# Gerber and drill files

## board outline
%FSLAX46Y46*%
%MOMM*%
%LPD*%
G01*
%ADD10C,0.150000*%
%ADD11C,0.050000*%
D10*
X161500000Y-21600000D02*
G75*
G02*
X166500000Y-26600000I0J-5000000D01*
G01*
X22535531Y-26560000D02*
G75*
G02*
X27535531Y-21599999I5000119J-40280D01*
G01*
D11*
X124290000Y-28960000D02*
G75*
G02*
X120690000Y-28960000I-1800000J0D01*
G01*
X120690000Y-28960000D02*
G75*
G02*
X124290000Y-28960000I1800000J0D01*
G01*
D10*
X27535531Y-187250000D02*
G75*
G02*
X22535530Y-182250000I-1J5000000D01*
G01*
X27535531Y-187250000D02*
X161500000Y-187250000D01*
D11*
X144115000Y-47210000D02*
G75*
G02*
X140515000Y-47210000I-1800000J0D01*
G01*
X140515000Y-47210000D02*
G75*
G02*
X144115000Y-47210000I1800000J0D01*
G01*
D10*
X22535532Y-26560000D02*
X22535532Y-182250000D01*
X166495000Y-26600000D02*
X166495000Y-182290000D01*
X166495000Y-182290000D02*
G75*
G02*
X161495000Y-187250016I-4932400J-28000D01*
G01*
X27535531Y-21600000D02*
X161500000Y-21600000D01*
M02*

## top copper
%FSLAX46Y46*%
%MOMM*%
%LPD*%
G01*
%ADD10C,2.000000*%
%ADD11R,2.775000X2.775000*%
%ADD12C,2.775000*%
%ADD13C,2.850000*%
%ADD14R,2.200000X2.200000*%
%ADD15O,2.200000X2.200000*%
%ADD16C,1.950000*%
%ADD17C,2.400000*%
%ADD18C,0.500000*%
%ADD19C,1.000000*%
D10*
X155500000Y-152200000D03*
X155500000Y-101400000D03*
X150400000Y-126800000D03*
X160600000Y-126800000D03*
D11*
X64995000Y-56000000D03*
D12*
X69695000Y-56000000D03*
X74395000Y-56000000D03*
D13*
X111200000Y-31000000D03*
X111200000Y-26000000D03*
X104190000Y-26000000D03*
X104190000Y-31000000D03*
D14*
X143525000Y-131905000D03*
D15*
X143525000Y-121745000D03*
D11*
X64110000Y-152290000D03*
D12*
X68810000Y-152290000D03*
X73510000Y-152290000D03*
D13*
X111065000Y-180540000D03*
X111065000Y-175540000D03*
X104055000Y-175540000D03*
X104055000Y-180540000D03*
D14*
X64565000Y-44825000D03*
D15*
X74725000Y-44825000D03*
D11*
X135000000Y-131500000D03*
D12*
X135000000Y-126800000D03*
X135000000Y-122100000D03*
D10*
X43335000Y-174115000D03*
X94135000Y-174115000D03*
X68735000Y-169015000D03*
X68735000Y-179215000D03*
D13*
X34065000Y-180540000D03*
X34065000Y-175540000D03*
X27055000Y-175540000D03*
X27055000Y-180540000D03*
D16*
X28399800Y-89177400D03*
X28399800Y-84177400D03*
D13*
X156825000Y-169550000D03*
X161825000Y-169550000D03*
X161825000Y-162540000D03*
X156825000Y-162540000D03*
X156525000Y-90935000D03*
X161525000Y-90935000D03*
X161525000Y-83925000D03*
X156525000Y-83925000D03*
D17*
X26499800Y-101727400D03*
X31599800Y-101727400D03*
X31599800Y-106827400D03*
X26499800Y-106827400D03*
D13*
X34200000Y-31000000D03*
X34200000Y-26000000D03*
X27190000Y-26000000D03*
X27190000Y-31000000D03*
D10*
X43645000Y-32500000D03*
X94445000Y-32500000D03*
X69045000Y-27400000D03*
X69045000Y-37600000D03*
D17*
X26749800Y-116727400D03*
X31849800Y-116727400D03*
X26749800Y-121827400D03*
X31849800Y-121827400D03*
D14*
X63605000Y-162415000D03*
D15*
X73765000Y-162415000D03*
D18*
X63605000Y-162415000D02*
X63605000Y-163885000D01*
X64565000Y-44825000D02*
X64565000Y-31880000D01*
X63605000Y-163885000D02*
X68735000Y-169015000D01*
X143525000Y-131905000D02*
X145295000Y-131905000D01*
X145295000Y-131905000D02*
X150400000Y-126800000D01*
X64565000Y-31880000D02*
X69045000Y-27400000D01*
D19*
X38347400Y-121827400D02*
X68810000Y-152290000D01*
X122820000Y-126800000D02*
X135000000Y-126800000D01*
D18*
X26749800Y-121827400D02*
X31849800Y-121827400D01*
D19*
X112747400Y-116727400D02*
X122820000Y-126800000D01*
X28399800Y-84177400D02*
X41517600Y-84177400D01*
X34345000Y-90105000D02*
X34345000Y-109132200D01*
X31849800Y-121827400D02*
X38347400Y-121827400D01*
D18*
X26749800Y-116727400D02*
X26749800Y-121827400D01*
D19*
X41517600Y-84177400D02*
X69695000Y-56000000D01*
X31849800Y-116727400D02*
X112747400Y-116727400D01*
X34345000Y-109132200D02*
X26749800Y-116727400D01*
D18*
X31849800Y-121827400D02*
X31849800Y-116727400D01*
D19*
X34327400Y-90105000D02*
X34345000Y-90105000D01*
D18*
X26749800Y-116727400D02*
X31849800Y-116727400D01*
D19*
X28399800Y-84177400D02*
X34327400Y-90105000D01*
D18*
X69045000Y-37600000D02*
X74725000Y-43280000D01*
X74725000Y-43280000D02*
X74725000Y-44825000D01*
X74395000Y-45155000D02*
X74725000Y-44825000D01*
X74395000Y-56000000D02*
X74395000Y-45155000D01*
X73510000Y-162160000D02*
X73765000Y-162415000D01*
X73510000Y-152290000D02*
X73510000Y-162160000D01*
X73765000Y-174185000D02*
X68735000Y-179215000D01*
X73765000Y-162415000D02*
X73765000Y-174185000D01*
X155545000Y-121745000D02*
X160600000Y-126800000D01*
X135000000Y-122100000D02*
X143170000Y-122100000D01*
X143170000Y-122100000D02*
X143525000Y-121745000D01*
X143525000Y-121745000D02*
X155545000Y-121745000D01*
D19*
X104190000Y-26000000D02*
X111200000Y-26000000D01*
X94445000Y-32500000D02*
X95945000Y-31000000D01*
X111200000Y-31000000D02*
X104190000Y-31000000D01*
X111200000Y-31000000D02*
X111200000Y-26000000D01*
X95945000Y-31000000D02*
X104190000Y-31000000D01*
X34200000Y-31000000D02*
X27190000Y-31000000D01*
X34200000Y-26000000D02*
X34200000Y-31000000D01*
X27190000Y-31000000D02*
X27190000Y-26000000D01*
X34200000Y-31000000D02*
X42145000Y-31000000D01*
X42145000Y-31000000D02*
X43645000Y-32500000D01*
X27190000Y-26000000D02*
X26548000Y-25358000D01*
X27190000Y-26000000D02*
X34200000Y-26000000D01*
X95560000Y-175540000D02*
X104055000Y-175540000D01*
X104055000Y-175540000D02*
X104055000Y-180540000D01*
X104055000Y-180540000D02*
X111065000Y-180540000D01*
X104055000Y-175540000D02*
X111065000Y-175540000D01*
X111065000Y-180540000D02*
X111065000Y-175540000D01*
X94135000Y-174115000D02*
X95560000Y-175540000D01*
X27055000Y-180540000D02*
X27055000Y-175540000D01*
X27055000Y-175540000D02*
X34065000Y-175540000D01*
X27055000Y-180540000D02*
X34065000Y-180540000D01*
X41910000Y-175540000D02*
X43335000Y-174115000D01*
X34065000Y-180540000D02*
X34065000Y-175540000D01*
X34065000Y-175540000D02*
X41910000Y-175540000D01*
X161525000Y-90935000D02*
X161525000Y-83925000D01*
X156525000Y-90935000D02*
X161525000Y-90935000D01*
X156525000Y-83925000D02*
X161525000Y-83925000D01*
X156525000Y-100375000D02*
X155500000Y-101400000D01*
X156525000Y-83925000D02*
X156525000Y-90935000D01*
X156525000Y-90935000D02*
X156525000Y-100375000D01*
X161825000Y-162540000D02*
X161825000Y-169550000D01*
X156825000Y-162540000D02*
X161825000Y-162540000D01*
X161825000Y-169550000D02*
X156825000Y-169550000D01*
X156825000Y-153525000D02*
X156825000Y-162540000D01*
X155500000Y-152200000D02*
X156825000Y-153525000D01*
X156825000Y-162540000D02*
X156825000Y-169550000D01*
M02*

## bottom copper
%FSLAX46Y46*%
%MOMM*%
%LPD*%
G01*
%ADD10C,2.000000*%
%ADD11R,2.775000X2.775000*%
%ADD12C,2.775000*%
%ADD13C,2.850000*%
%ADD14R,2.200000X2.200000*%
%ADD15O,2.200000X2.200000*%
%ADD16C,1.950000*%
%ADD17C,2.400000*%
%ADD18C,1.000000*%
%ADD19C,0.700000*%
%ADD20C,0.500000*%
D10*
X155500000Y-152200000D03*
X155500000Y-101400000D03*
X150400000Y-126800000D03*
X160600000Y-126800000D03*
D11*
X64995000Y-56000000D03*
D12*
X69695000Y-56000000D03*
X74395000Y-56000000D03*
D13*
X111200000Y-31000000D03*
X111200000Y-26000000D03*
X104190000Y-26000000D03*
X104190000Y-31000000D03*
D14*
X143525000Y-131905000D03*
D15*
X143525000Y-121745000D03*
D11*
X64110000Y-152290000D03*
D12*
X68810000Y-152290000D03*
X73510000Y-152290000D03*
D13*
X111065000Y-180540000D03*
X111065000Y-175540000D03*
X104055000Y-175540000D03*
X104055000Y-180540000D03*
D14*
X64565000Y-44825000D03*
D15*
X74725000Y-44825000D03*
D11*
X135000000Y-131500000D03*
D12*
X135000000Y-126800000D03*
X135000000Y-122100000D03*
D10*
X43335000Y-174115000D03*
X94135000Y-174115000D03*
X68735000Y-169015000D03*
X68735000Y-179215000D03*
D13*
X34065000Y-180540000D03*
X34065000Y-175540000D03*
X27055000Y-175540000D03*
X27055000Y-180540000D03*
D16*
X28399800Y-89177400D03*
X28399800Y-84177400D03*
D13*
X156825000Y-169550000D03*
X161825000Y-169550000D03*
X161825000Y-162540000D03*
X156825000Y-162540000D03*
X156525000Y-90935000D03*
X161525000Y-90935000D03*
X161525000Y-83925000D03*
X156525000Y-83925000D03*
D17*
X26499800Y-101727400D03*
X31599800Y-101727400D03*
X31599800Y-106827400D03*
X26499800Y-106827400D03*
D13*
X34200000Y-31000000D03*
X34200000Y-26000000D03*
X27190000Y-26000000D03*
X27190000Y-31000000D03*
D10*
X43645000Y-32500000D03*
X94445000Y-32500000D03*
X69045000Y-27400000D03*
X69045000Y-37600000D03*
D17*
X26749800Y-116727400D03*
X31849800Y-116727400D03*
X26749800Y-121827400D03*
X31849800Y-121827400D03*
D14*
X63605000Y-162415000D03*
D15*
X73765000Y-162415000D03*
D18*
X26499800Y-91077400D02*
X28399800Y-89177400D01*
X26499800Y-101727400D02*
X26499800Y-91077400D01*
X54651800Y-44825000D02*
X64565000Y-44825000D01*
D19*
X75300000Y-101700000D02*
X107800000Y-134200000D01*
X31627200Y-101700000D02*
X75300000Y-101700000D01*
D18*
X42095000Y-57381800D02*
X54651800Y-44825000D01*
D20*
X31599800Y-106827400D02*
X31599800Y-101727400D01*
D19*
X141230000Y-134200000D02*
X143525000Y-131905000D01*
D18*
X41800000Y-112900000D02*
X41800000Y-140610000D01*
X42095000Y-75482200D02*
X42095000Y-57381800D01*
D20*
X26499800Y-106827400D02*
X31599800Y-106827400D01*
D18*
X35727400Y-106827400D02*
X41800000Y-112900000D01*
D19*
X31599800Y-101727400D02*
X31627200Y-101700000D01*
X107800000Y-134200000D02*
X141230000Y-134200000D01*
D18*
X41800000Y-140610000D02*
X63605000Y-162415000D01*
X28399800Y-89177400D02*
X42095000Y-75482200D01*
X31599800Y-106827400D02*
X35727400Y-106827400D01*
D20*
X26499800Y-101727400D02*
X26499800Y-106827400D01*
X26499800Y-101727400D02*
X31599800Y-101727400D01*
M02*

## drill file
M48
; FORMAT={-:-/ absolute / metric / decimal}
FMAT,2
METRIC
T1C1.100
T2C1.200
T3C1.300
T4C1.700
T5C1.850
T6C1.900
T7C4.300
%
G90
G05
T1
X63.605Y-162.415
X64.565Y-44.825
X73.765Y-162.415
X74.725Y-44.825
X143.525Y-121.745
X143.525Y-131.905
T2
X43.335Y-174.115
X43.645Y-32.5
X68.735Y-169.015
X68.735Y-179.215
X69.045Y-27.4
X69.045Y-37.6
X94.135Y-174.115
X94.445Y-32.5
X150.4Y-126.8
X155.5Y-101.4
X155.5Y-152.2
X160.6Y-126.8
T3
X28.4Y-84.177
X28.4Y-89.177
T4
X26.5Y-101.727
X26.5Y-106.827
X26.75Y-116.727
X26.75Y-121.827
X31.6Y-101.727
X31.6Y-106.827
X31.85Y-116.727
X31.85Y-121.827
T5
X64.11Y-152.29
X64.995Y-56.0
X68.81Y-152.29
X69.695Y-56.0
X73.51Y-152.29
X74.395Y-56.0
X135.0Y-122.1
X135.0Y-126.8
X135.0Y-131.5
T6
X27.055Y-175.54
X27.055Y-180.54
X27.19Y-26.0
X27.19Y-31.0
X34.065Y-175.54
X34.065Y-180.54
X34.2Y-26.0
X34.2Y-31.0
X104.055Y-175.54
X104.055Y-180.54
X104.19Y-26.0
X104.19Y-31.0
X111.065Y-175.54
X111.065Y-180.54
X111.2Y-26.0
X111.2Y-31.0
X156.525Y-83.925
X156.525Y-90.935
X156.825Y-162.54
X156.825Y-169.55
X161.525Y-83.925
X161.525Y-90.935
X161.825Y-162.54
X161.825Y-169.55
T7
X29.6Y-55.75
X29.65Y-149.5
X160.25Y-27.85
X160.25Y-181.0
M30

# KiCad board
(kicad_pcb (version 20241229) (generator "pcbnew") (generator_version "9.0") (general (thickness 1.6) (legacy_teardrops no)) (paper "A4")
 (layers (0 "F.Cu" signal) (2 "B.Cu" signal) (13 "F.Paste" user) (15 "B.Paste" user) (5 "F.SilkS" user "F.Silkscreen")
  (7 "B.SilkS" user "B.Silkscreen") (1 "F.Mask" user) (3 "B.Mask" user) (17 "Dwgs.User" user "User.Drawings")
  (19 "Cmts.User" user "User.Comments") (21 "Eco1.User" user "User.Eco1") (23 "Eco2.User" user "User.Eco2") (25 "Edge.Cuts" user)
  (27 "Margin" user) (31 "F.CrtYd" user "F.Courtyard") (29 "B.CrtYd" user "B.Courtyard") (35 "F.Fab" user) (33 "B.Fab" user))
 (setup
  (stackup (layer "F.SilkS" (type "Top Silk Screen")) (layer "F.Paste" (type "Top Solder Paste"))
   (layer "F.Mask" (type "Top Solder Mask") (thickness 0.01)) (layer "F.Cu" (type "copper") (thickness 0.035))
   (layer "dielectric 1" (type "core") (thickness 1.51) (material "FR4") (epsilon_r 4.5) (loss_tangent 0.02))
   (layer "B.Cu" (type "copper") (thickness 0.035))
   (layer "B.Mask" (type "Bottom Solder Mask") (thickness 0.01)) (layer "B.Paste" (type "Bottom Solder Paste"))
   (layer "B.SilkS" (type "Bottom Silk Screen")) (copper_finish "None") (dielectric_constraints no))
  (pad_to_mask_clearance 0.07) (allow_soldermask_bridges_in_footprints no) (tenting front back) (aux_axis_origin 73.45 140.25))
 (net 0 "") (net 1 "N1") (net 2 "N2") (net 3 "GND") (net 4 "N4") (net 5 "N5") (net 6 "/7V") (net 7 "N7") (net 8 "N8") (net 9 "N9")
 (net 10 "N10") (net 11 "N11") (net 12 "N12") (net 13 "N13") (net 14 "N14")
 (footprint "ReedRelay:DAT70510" (layer "F.Cu") (at 155.5 126.8 90)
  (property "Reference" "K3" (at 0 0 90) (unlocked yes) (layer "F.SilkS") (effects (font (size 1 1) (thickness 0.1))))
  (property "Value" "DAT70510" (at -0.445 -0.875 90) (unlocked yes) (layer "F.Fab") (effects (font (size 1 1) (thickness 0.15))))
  (pad "1" thru_hole circle (at -25.4 0 90) (size 2 2) (drill 1.2) (layers "*.Cu" "*.Mask") (remove_unused_layers no) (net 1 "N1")
   (solder_mask_margin 0.075))
  (pad "2" thru_hole circle (at 25.4 0 90) (size 2 2) (drill 1.2) (layers "*.Cu" "*.Mask") (remove_unused_layers no) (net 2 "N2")
   (solder_mask_margin 0.075))
  (pad "3" thru_hole circle (at 0 -5.1 90) (size 2 2) (drill 1.2) (layers "*.Cu" "*.Mask") (remove_unused_layers no) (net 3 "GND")
   (solder_mask_margin 0.075))
  (pad "4" thru_hole circle (at 0 5.1 90) (size 2 2) (drill 1.2) (layers "*.Cu" "*.Mask") (remove_unused_layers no) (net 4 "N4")
   (solder_mask_margin 0.075)))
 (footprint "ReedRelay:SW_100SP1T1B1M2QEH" (layer "F.Cu") (at 69.695 56)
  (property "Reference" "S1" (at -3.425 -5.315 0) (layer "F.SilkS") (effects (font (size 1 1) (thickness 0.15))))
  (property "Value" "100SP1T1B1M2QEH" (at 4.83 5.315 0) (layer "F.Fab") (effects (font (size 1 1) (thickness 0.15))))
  (pad "1" thru_hole rect (at -4.7 0) (size 2.775 2.775) (drill 1.85) (layers "*.Cu" "*.Mask") (remove_unused_layers no) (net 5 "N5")
   (solder_mask_margin 0.102))
  (pad "2" thru_hole circle (at 0 0) (size 2.775 2.775) (drill 1.85) (layers "*.Cu" "*.Mask") (remove_unused_layers no) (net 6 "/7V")
   (solder_mask_margin 0.102))
  (pad "3" thru_hole circle (at 4.7 0) (size 2.775 2.775) (drill 1.85) (layers "*.Cu" "*.Mask") (remove_unused_layers no) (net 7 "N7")
   (solder_mask_margin 0.102)))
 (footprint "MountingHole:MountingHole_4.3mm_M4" (layer "F.Cu") (at 160.25 181)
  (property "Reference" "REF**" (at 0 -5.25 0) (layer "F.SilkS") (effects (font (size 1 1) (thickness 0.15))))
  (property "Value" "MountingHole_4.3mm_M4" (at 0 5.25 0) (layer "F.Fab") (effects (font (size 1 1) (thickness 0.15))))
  (pad "" np_thru_hole circle (at 0 0) (size 4.3 4.3) (drill 4.3) (layers "*.Cu" "*.Mask")))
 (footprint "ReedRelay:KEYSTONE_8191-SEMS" (layer "F.Cu") (at 107.695 28.5 90)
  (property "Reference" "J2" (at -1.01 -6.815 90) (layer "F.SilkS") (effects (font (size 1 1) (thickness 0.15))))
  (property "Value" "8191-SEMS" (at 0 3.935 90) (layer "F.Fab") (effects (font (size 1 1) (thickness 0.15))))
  (pad "1_1" thru_hole circle (at -2.5 3.505 90) (size 2.85 2.85) (drill 1.9) (layers "*.Cu" "*.Mask") (remove_unused_layers no)
   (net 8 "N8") (solder_mask_margin 0.102))
  (pad "1_2" thru_hole circle (at 2.5 3.505 90) (size 2.85 2.85) (drill 1.9) (layers "*.Cu" "*.Mask") (remove_unused_layers no) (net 8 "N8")
   (solder_mask_margin 0.102))
  (pad "1_3" thru_hole circle (at 2.5 -3.505 90) (size 2.85 2.85) (drill 1.9) (layers "*.Cu" "*.Mask") (remove_unused_layers no)
   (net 8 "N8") (solder_mask_margin 0.102))
  (pad "1_4" thru_hole circle (at -2.5 -3.505 90) (size 2.85 2.85) (drill 1.9) (layers "*.Cu" "*.Mask") (remove_unused_layers no)
   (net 8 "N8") (solder_mask_margin 0.102)))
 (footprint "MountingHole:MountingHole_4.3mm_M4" (layer "F.Cu") (at 160.25 27.85)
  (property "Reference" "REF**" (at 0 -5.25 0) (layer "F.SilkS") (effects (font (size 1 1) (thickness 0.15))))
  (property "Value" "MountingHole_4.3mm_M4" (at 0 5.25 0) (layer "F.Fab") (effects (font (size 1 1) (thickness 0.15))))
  (pad "" np_thru_hole circle (at 0 0) (size 4.3 4.3) (drill 4.3) (layers "*.Cu" "*.Mask")))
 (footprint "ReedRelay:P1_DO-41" (layer "F.Cu") (at 143.525 131.905 90)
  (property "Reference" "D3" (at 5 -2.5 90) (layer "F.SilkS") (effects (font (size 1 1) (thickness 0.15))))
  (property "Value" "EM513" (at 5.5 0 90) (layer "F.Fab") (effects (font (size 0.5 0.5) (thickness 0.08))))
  (pad "1" thru_hole rect (at 0 0 90) (size 2.2 2.2) (drill 1.1) (layers "*.Cu" "*.Mask") (remove_unused_layers no) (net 3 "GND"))
  (pad "2" thru_hole oval (at 10.16 0 90) (size 2.2 2.2) (drill 1.1) (layers "*.Cu" "*.Mask") (remove_unused_layers no) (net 4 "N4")))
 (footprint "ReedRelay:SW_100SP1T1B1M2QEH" (layer "F.Cu") (at 68.81 152.29)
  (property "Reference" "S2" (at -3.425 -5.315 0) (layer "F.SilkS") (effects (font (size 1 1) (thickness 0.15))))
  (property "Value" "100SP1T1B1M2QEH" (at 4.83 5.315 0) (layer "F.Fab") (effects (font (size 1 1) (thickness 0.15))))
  (pad "1" thru_hole rect (at -4.7 0) (size 2.775 2.775) (drill 1.85) (layers "*.Cu" "*.Mask") (remove_unused_layers no) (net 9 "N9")
   (solder_mask_margin 0.102))
  (pad "2" thru_hole circle (at 0 0) (size 2.775 2.775) (drill 1.85) (layers "*.Cu" "*.Mask") (remove_unused_layers no) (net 6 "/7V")
   (solder_mask_margin 0.102))
  (pad "3" thru_hole circle (at 4.7 0) (size 2.775 2.775) (drill 1.85) (layers "*.Cu" "*.Mask") (remove_unused_layers no) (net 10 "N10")
   (solder_mask_margin 0.102)))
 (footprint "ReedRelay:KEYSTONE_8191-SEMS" (layer "F.Cu") (at 107.56 178.04 90)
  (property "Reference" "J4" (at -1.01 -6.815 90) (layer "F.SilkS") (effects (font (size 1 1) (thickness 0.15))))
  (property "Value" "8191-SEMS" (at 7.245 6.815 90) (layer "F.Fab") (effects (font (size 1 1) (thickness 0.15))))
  (pad "1_1" thru_hole circle (at -2.5 3.505 90) (size 2.85 2.85) (drill 1.9) (layers "*.Cu" "*.Mask") (remove_unused_layers no)
   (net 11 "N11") (solder_mask_margin 0.102))
  (pad "1_2" thru_hole circle (at 2.5 3.505 90) (size 2.85 2.85) (drill 1.9) (layers "*.Cu" "*.Mask") (remove_unused_layers no)
   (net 11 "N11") (solder_mask_margin 0.102))
  (pad "1_3" thru_hole circle (at 2.5 -3.505 90) (size 2.85 2.85) (drill 1.9) (layers "*.Cu" "*.Mask") (remove_unused_layers no)
   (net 11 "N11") (solder_mask_margin 0.102))
  (pad "1_4" thru_hole circle (at -2.5 -3.505 90) (size 2.85 2.85) (drill 1.9) (layers "*.Cu" "*.Mask") (remove_unused_layers no)
   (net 11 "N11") (solder_mask_margin 0.102)))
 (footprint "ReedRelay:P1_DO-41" (layer "F.Cu") (at 64.565 44.825)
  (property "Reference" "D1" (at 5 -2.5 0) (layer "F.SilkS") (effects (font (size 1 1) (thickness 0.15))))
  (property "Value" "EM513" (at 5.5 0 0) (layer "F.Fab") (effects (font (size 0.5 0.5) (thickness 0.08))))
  (pad "1" thru_hole rect (at 0 0) (size 2.2 2.2) (drill 1.1) (layers "*.Cu" "*.Mask") (remove_unused_layers no) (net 3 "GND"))
  (pad "2" thru_hole oval (at 10.16 0) (size 2.2 2.2) (drill 1.1) (layers "*.Cu" "*.Mask") (remove_unused_layers no) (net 7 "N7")))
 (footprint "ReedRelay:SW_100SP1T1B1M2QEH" (layer "F.Cu") (at 135 126.8 90)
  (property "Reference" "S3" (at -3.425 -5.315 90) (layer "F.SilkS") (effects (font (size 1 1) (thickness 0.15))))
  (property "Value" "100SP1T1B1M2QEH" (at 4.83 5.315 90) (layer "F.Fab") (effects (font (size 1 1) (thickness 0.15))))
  (pad "1" thru_hole rect (at -4.7 0 90) (size 2.775 2.775) (drill 1.85) (layers "*.Cu" "*.Mask") (remove_unused_layers no) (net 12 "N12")
   (solder_mask_margin 0.102))
  (pad "2" thru_hole circle (at 0 0 90) (size 2.775 2.775) (drill 1.85) (layers "*.Cu" "*.Mask") (remove_unused_layers no) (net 6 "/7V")
   (solder_mask_margin 0.102))
  (pad "3" thru_hole circle (at 4.7 0 90) (size 2.775 2.775) (drill 1.85) (layers "*.Cu" "*.Mask") (remove_unused_layers no) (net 4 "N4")
   (solder_mask_margin 0.102)))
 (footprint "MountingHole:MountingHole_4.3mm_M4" (layer "F.Cu") (at 29.65 149.5 90)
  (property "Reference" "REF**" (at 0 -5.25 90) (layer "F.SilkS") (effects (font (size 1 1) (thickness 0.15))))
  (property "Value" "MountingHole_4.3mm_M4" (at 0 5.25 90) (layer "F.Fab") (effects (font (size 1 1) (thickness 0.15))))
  (pad "" np_thru_hole circle (at 0 0 90) (size 4.3 4.3) (drill 4.3) (layers "*.Cu" "*.Mask")))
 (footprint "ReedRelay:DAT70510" (layer "F.Cu") (at 68.735 174.115)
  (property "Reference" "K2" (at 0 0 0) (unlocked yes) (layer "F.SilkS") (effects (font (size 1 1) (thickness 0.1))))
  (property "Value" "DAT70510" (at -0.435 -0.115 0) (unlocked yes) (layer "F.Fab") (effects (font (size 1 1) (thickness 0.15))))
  (pad "1" thru_hole circle (at -25.4 0) (size 2 2) (drill 1.2) (layers "*.Cu" "*.Mask") (remove_unused_layers no) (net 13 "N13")
   (solder_mask_margin 0.075))
  (pad "2" thru_hole circle (at 25.4 0) (size 2 2) (drill 1.2) (layers "*.Cu" "*.Mask") (remove_unused_layers no) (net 11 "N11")
   (solder_mask_margin 0.075))
  (pad "3" thru_hole circle (at 0 -5.1) (size 2 2) (drill 1.2) (layers "*.Cu" "*.Mask") (remove_unused_layers no) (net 3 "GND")
   (solder_mask_margin 0.075))
  (pad "4" thru_hole circle (at 0 5.1) (size 2 2) (drill 1.2) (layers "*.Cu" "*.Mask") (remove_unused_layers no) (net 10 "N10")
   (solder_mask_margin 0.075)))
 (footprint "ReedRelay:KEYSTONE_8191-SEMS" (layer "F.Cu") (at 30.56 178.04 90)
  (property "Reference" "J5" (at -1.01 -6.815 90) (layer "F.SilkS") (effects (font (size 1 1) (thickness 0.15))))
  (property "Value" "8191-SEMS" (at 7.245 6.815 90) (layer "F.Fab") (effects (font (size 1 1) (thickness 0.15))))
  (pad "1_1" thru_hole circle (at -2.5 3.505 90) (size 2.85 2.85) (drill 1.9) (layers "*.Cu" "*.Mask") (remove_unused_layers no)
   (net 13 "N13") (solder_mask_margin 0.102))
  (pad "1_2" thru_hole circle (at 2.5 3.505 90) (size 2.85 2.85) (drill 1.9) (layers "*.Cu" "*.Mask") (remove_unused_layers no)
   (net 13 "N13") (solder_mask_margin 0.102))
  (pad "1_3" thru_hole circle (at 2.5 -3.505 90) (size 2.85 2.85) (drill 1.9) (layers "*.Cu" "*.Mask") (remove_unused_layers no)
   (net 13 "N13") (solder_mask_margin 0.102))
  (pad "1_4" thru_hole circle (at -2.5 -3.505 90) (size 2.85 2.85) (drill 1.9) (layers "*.Cu" "*.Mask") (remove_unused_layers no)
   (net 13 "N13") (solder_mask_margin 0.102)))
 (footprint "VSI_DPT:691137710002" (layer "F.Cu") (at 28.3998 86.6774 90)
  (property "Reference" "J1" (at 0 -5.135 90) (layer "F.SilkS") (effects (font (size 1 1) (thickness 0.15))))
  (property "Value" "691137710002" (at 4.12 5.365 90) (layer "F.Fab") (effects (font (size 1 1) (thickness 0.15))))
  (pad "1" thru_hole circle (at -2.5 0 90) (size 1.95 1.95) (drill 1.3) (layers "*.Cu" "*.Mask") (remove_unused_layers no) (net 3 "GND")
   (solder_mask_margin 0.102))
  (pad "2" thru_hole circle (at 2.5 0 90) (size 1.95 1.95) (drill 1.3) (layers "*.Cu" "*.Mask") (remove_unused_layers no) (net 6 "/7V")
   (solder_mask_margin 0.102)))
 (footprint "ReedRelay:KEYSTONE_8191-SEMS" (layer "F.Cu") (at 159.325 166.045)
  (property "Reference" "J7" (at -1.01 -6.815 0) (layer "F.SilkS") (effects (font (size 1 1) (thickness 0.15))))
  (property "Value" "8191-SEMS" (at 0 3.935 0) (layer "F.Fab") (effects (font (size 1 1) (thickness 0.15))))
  (pad "1_1" thru_hole circle (at -2.5 3.505) (size 2.85 2.85) (drill 1.9) (layers "*.Cu" "*.Mask") (remove_unused_layers no) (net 1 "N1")
   (solder_mask_margin 0.102))
  (pad "1_2" thru_hole circle (at 2.5 3.505) (size 2.85 2.85) (drill 1.9) (layers "*.Cu" "*.Mask") (remove_unused_layers no) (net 1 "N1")
   (solder_mask_margin 0.102))
  (pad "1_3" thru_hole circle (at 2.5 -3.505) (size 2.85 2.85) (drill 1.9) (layers "*.Cu" "*.Mask") (remove_unused_layers no) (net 1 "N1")
   (solder_mask_margin 0.102))
  (pad "1_4" thru_hole circle (at -2.5 -3.505) (size 2.85 2.85) (drill 1.9) (layers "*.Cu" "*.Mask") (remove_unused_layers no) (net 1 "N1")
   (solder_mask_margin 0.102)))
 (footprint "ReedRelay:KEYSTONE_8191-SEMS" (layer "F.Cu") (at 159.025 87.43)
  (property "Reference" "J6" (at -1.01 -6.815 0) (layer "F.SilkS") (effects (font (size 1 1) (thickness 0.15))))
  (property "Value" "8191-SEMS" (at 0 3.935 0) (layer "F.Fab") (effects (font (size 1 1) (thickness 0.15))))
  (pad "1_1" thru_hole circle (at -2.5 3.505) (size 2.85 2.85) (drill 1.9) (layers "*.Cu" "*.Mask") (remove_unused_layers no) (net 2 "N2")
   (solder_mask_margin 0.102))
  (pad "1_2" thru_hole circle (at 2.5 3.505) (size 2.85 2.85) (drill 1.9) (layers "*.Cu" "*.Mask") (remove_unused_layers no) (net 2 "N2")
   (solder_mask_margin 0.102))
  (pad "1_3" thru_hole circle (at 2.5 -3.505) (size 2.85 2.85) (drill 1.9) (layers "*.Cu" "*.Mask") (remove_unused_layers no) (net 2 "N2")
   (solder_mask_margin 0.102))
  (pad "1_4" thru_hole circle (at -2.5 -3.505) (size 2.85 2.85) (drill 1.9) (layers "*.Cu" "*.Mask") (remove_unused_layers no) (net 2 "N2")
   (solder_mask_margin 0.102)))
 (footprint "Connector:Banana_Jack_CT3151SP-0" (layer "F.Cu") (at 29.0498 104.2774 90)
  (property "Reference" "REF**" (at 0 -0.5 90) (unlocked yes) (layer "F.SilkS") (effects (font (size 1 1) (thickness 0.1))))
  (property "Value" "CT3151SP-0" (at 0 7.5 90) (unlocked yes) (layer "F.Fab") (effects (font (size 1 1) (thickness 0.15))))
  (pad "1" thru_hole circle (at 2.55 -2.55 90) (size 2.4 2.4) (drill 1.7) (layers "*.Cu" "*.Mask") (remove_unused_layers no) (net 3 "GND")
   (solder_mask_margin 0.075))
  (pad "2" thru_hole circle (at 2.55 2.55 90) (size 2.4 2.4) (drill 1.7) (layers "*.Cu" "*.Mask") (remove_unused_layers no) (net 3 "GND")
   (solder_mask_margin 0.075))
  (pad "3" thru_hole circle (at -2.55 2.55 90) (size 2.4 2.4) (drill 1.7) (layers "*.Cu" "*.Mask") (remove_unused_layers no) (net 3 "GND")
   (solder_mask_margin 0.075))
  (pad "4" thru_hole circle (at -2.55 -2.55 90) (size 2.4 2.4) (drill 1.7) (layers "*.Cu" "*.Mask") (remove_unused_layers no) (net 3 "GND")
   (solder_mask_margin 0.075)))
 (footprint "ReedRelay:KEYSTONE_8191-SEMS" (layer "F.Cu") (at 30.695 28.5 90)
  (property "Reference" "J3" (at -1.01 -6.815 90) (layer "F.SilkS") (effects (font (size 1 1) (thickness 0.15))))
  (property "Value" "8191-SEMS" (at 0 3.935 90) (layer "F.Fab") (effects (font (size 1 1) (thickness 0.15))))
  (pad "1_1" thru_hole circle (at -2.5 3.505 90) (size 2.85 2.85) (drill 1.9) (layers "*.Cu" "*.Mask") (remove_unused_layers no)
   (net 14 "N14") (solder_mask_margin 0.102))
  (pad "1_2" thru_hole circle (at 2.5 3.505 90) (size 2.85 2.85) (drill 1.9) (layers "*.Cu" "*.Mask") (remove_unused_layers no)
   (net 14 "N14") (solder_mask_margin 0.102))
  (pad "1_3" thru_hole circle (at 2.5 -3.505 90) (size 2.85 2.85) (drill 1.9) (layers "*.Cu" "*.Mask") (remove_unused_layers no)
   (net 14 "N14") (solder_mask_margin 0.102))
  (pad "1_4" thru_hole circle (at -2.5 -3.505 90) (size 2.85 2.85) (drill 1.9) (layers "*.Cu" "*.Mask") (remove_unused_layers no)
   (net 14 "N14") (solder_mask_margin 0.102)))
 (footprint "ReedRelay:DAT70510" (layer "F.Cu") (at 69.045 32.5)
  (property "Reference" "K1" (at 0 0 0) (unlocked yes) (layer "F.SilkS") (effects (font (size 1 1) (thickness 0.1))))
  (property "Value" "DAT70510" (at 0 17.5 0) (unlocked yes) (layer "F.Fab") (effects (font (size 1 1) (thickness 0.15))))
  (pad "1" thru_hole circle (at -25.4 0) (size 2 2) (drill 1.2) (layers "*.Cu" "*.Mask") (remove_unused_layers no) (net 14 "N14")
   (solder_mask_margin 0.075))
  (pad "2" thru_hole circle (at 25.4 0) (size 2 2) (drill 1.2) (layers "*.Cu" "*.Mask") (remove_unused_layers no) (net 8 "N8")
   (solder_mask_margin 0.075))
  (pad "3" thru_hole circle (at 0 -5.1) (size 2 2) (drill 1.2) (layers "*.Cu" "*.Mask") (remove_unused_layers no) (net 3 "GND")
   (solder_mask_margin 0.075))
  (pad "4" thru_hole circle (at 0 5.1) (size 2 2) (drill 1.2) (layers "*.Cu" "*.Mask") (remove_unused_layers no) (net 7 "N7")
   (solder_mask_margin 0.075)))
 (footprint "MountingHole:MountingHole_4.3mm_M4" (layer "F.Cu") (at 29.6 55.75 90)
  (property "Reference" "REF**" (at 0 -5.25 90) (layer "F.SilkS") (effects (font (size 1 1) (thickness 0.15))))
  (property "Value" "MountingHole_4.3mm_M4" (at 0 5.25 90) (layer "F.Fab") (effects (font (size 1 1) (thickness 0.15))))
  (pad "" np_thru_hole circle (at 0 0 90) (size 4.3 4.3) (drill 4.3) (layers "*.Cu" "*.Mask")))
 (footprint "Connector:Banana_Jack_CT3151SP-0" (layer "F.Cu") (at 29.2998 119.2774 90)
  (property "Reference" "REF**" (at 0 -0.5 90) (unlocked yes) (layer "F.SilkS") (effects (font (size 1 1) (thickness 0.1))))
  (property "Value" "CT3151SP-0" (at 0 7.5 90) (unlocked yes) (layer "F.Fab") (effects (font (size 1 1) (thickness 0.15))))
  (pad "1" thru_hole circle (at 2.55 -2.55 90) (size 2.4 2.4) (drill 1.7) (layers "*.Cu" "*.Mask") (remove_unused_layers no) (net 6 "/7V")
   (solder_mask_margin 0.075))
  (pad "2" thru_hole circle (at 2.55 2.55 90) (size 2.4 2.4) (drill 1.7) (layers "*.Cu" "*.Mask") (remove_unused_layers no) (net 6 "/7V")
   (solder_mask_margin 0.075))
  (pad "3" thru_hole circle (at -2.55 -2.55 90) (size 2.4 2.4) (drill 1.7) (layers "*.Cu" "*.Mask") (remove_unused_layers no) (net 6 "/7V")
   (solder_mask_margin 0.075))
  (pad "3" thru_hole circle (at -2.55 2.55 90) (size 2.4 2.4) (drill 1.7) (layers "*.Cu" "*.Mask") (remove_unused_layers no) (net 6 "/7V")
   (solder_mask_margin 0.075)))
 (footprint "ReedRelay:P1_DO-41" (layer "F.Cu") (at 63.605 162.415)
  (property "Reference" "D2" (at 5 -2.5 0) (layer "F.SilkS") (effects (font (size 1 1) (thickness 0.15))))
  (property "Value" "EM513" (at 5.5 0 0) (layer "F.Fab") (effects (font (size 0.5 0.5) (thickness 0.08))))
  (pad "1" thru_hole rect (at 0 0) (size 2.2 2.2) (drill 1.1) (layers "*.Cu" "*.Mask") (remove_unused_layers no) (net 3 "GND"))
  (pad "2" thru_hole oval (at 10.16 0) (size 2.2 2.2) (drill 1.1) (layers "*.Cu" "*.Mask") (remove_unused_layers no) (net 10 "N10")))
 (gr_arc (start 161.5 21.6) (mid 165.035534 23.064466) (end 166.5 26.6) (stroke (width 0.15) (type solid)) (layer "Edge.Cuts"))
 (gr_arc (start 22.535531 26.56) (mid 24.014145 23.050377) (end 27.535531 21.6) (stroke (width 0.15) (type solid)) (layer "Edge.Cuts"))
 (gr_circle (center 122.49 28.96) (end 124.29 28.96) (stroke (width 0.05) (type solid)) (fill no) (layer "Edge.Cuts"))
 (gr_arc (start 27.535531 187.25) (mid 23.999996 185.785535) (end 22.535531 182.25) (stroke (width 0.15) (type solid)) (layer "Edge.Cuts"))
 (gr_line (start 27.535531 187.25) (end 161.5 187.25) (stroke (width 0.15) (type solid)) (layer "Edge.Cuts"))
 (gr_circle (center 142.315 47.21) (end 144.115 47.21) (stroke (width 0.05) (type solid)) (fill no) (layer "Edge.Cuts"))
 (gr_line (start 22.535532 26.56) (end 22.535532 182.25) (stroke (width 0.15) (type solid)) (layer "Edge.Cuts"))
 (gr_line (start 166.495 26.6) (end 166.495 182.29) (stroke (width 0.15) (type solid)) (layer "Edge.Cuts"))
 (gr_arc (start 166.495 182.29) (mid 165.030535 185.825535) (end 161.495 187.25) (stroke (width 0.15) (type solid)) (layer "Edge.Cuts"))
 (gr_line (start 27.535531 21.6) (end 161.5 21.6) (stroke (width 0.15) (type solid)) (layer "Edge.Cuts"))
 (segment (start 63.605 162.415) (end 63.605 163.885) (width 0.5) (layer "F.Cu") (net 3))
 (segment (start 64.565 44.825) (end 64.565 31.88) (width 0.5) (layer "F.Cu") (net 3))
 (segment (start 63.605 163.885) (end 68.735 169.015) (width 0.5) (layer "F.Cu") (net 3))
 (segment (start 143.525 131.905) (end 145.295 131.905) (width 0.5) (layer "F.Cu") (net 3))
 (segment (start 145.295 131.905) (end 150.4 126.8) (width 0.5) (layer "F.Cu") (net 3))
 (segment (start 64.565 31.88) (end 69.045 27.4) (width 0.5) (layer "F.Cu") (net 3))
 (segment (start 26.4998 91.0774) (end 28.3998 89.1774) (width 1) (layer "B.Cu") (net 3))
 (segment (start 26.4998 101.7274) (end 26.4998 91.0774) (width 1) (layer "B.Cu") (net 3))
 (segment (start 54.6518 44.825) (end 64.565 44.825) (width 1) (layer "B.Cu") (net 3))
 (segment (start 75.3 101.7) (end 107.8 134.2) (width 0.7) (layer "B.Cu") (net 3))
 (segment (start 31.6272 101.7) (end 75.3 101.7) (width 0.7) (layer "B.Cu") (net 3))
 (segment (start 42.095 57.3818) (end 54.6518 44.825) (width 1) (layer "B.Cu") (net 3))
 (segment (start 31.5998 106.8274) (end 31.5998 101.7274) (width 0.5) (layer "B.Cu") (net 3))
 (segment (start 141.23 134.2) (end 143.525 131.905) (width 0.7) (layer "B.Cu") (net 3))
 (segment (start 41.8 112.9) (end 41.8 140.61) (width 1) (layer "B.Cu") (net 3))
 (segment (start 42.095 75.4822) (end 42.095 57.3818) (width 1) (layer "B.Cu") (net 3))
 (segment (start 26.4998 106.8274) (end 31.5998 106.8274) (width 0.5) (layer "B.Cu") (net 3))
 (segment (start 35.7274 106.8274) (end 41.8 112.9) (width 1) (layer "B.Cu") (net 3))
 (segment (start 31.5998 101.7274) (end 31.6272 101.7) (width 0.7) (layer "B.Cu") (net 3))
 (segment (start 107.8 134.2) (end 141.23 134.2) (width 0.7) (layer "B.Cu") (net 3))
 (segment (start 41.8 140.61) (end 63.605 162.415) (width 1) (layer "B.Cu") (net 3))
 (segment (start 28.3998 89.1774) (end 42.095 75.4822) (width 1) (layer "B.Cu") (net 3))
 (segment (start 31.5998 106.8274) (end 35.7274 106.8274) (width 1) (layer "B.Cu") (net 3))
 (segment (start 26.4998 101.7274) (end 26.4998 106.8274) (width 0.5) (layer "B.Cu") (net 3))
 (segment (start 26.4998 101.7274) (end 31.5998 101.7274) (width 0.5) (layer "B.Cu") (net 3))
 (segment (start 38.3474 121.8274) (end 68.81 152.29) (width 1) (layer "F.Cu") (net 6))
 (segment (start 122.82 126.8) (end 135 126.8) (width 1) (layer "F.Cu") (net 6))
 (segment (start 26.7498 121.8274) (end 31.8498 121.8274) (width 0.5) (layer "F.Cu") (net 6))
 (segment (start 112.7474 116.7274) (end 122.82 126.8) (width 1) (layer "F.Cu") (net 6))
 (segment (start 28.3998 84.1774) (end 41.5176 84.1774) (width 1) (layer "F.Cu") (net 6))
 (segment (start 34.345 90.105) (end 34.345 109.1322) (width 1) (layer "F.Cu") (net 6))
 (segment (start 31.8498 121.8274) (end 38.3474 121.8274) (width 1) (layer "F.Cu") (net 6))
 (segment (start 26.7498 116.7274) (end 26.7498 121.8274) (width 0.5) (layer "F.Cu") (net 6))
 (segment (start 41.5176 84.1774) (end 69.695 56) (width 1) (layer "F.Cu") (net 6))
 (segment (start 31.8498 116.7274) (end 112.7474 116.7274) (width 1) (layer "F.Cu") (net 6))
 (segment (start 34.345 109.1322) (end 26.7498 116.7274) (width 1) (layer "F.Cu") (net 6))
 (segment (start 31.8498 121.8274) (end 31.8498 116.7274) (width 0.5) (layer "F.Cu") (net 6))
 (segment (start 34.3274 90.105) (end 34.345 90.105) (width 1) (layer "F.Cu") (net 6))
 (segment (start 26.7498 116.7274) (end 31.8498 116.7274) (width 0.5) (layer "F.Cu") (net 6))
 (segment (start 28.3998 84.1774) (end 34.3274 90.105) (width 1) (layer "F.Cu") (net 6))
 (segment (start 69.045 37.6) (end 74.725 43.28) (width 0.5) (layer "F.Cu") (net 7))
 (segment (start 74.725 43.28) (end 74.725 44.825) (width 0.5) (layer "F.Cu") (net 7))
 (segment (start 74.395 45.155) (end 74.725 44.825) (width 0.5) (layer "F.Cu") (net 7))
 (segment (start 74.395 56) (end 74.395 45.155) (width 0.5) (layer "F.Cu") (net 7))
 (segment (start 73.51 162.16) (end 73.765 162.415) (width 0.5) (layer "F.Cu") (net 10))
 (segment (start 73.51 152.29) (end 73.51 162.16) (width 0.5) (layer "F.Cu") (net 10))
 (segment (start 73.765 174.185) (end 68.735 179.215) (width 0.5) (layer "F.Cu") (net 10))
 (segment (start 73.765 162.415) (end 73.765 174.185) (width 0.5) (layer "F.Cu") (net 10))
 (segment (start 155.545 121.745) (end 160.6 126.8) (width 0.5) (layer "F.Cu") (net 4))
 (segment (start 135 122.1) (end 143.17 122.1) (width 0.5) (layer "F.Cu") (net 4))
 (segment (start 143.17 122.1) (end 143.525 121.745) (width 0.5) (layer "F.Cu") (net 4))
 (segment (start 143.525 121.745) (end 155.545 121.745) (width 0.5) (layer "F.Cu") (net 4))
 (segment (start 104.19 26) (end 111.2 26) (width 1) (layer "F.Cu") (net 8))
 (segment (start 94.445 32.5) (end 95.945 31) (width 1) (layer "F.Cu") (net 8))
 (segment (start 111.2 31) (end 104.19 31) (width 1) (layer "F.Cu") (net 8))
 (segment (start 111.2 31) (end 111.2 26) (width 1) (layer "F.Cu") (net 8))
 (segment (start 95.945 31) (end 104.19 31) (width 1) (layer "F.Cu") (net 8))
 (segment (start 34.2 31) (end 27.19 31) (width 1) (layer "F.Cu") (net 14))
 (segment (start 34.2 26) (end 34.2 31) (width 1) (layer "F.Cu") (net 14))
 (segment (start 27.19 31) (end 27.19 26) (width 1) (layer "F.Cu") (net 14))
 (segment (start 34.2 31) (end 42.145 31) (width 1) (layer "F.Cu") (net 14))
 (segment (start 42.145 31) (end 43.645 32.5) (width 1) (layer "F.Cu") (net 14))
 (segment (start 27.19 26) (end 26.548 25.358) (width 1) (layer "F.Cu") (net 14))
 (segment (start 27.19 26) (end 34.2 26) (width 1) (layer "F.Cu") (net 14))
 (segment (start 95.56 175.54) (end 104.055 175.54) (width 1) (layer "F.Cu") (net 11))
 (segment (start 104.055 175.54) (end 104.055 180.54) (width 1) (layer "F.Cu") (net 11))
 (segment (start 104.055 180.54) (end 111.065 180.54) (width 1) (layer "F.Cu") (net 11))
 (segment (start 104.055 175.54) (end 111.065 175.54) (width 1) (layer "F.Cu") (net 11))
 (segment (start 111.065 180.54) (end 111.065 175.54) (width 1) (layer "F.Cu") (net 11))
 (segment (start 94.135 174.115) (end 95.56 175.54) (width 1) (layer "F.Cu") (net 11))
 (segment (start 27.055 180.54) (end 27.055 175.54) (width 1) (layer "F.Cu") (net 13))
 (segment (start 27.055 175.54) (end 34.065 175.54) (width 1) (layer "F.Cu") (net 13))
 (segment (start 27.055 180.54) (end 34.065 180.54) (width 1) (layer "F.Cu") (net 13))
 (segment (start 41.91 175.54) (end 43.335 174.115) (width 1) (layer "F.Cu") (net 13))
 (segment (start 34.065 180.54) (end 34.065 175.54) (width 1) (layer "F.Cu") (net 13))
 (segment (start 34.065 175.54) (end 41.91 175.54) (width 1) (layer "F.Cu") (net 13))
 (segment (start 161.525 90.935) (end 161.525 83.925) (width 1) (layer "F.Cu") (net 2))
 (segment (start 156.525 90.935) (end 161.525 90.935) (width 1) (layer "F.Cu") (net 2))
 (segment (start 156.525 83.925) (end 161.525 83.925) (width 1) (layer "F.Cu") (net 2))
 (segment (start 156.525 100.375) (end 155.5 101.4) (width 1) (layer "F.Cu") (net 2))
 (segment (start 156.525 83.925) (end 156.525 90.935) (width 1) (layer "F.Cu") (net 2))
 (segment (start 156.525 90.935) (end 156.525 100.375) (width 1) (layer "F.Cu") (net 2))
 (segment (start 161.825 162.54) (end 161.825 169.55) (width 1) (layer "F.Cu") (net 1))
 (segment (start 156.825 162.54) (end 161.825 162.54) (width 1) (layer "F.Cu") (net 1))
 (segment (start 161.825 169.55) (end 156.825 169.55) (width 1) (layer "F.Cu") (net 1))
 (segment (start 156.825 153.525) (end 156.825 162.54) (width 1) (layer "F.Cu") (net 1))
 (segment (start 155.5 152.2) (end 156.825 153.525) (width 1) (layer "F.Cu") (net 1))
 (segment (start 156.825 162.54) (end 156.825 169.55) (width 1) (layer "F.Cu") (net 1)))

